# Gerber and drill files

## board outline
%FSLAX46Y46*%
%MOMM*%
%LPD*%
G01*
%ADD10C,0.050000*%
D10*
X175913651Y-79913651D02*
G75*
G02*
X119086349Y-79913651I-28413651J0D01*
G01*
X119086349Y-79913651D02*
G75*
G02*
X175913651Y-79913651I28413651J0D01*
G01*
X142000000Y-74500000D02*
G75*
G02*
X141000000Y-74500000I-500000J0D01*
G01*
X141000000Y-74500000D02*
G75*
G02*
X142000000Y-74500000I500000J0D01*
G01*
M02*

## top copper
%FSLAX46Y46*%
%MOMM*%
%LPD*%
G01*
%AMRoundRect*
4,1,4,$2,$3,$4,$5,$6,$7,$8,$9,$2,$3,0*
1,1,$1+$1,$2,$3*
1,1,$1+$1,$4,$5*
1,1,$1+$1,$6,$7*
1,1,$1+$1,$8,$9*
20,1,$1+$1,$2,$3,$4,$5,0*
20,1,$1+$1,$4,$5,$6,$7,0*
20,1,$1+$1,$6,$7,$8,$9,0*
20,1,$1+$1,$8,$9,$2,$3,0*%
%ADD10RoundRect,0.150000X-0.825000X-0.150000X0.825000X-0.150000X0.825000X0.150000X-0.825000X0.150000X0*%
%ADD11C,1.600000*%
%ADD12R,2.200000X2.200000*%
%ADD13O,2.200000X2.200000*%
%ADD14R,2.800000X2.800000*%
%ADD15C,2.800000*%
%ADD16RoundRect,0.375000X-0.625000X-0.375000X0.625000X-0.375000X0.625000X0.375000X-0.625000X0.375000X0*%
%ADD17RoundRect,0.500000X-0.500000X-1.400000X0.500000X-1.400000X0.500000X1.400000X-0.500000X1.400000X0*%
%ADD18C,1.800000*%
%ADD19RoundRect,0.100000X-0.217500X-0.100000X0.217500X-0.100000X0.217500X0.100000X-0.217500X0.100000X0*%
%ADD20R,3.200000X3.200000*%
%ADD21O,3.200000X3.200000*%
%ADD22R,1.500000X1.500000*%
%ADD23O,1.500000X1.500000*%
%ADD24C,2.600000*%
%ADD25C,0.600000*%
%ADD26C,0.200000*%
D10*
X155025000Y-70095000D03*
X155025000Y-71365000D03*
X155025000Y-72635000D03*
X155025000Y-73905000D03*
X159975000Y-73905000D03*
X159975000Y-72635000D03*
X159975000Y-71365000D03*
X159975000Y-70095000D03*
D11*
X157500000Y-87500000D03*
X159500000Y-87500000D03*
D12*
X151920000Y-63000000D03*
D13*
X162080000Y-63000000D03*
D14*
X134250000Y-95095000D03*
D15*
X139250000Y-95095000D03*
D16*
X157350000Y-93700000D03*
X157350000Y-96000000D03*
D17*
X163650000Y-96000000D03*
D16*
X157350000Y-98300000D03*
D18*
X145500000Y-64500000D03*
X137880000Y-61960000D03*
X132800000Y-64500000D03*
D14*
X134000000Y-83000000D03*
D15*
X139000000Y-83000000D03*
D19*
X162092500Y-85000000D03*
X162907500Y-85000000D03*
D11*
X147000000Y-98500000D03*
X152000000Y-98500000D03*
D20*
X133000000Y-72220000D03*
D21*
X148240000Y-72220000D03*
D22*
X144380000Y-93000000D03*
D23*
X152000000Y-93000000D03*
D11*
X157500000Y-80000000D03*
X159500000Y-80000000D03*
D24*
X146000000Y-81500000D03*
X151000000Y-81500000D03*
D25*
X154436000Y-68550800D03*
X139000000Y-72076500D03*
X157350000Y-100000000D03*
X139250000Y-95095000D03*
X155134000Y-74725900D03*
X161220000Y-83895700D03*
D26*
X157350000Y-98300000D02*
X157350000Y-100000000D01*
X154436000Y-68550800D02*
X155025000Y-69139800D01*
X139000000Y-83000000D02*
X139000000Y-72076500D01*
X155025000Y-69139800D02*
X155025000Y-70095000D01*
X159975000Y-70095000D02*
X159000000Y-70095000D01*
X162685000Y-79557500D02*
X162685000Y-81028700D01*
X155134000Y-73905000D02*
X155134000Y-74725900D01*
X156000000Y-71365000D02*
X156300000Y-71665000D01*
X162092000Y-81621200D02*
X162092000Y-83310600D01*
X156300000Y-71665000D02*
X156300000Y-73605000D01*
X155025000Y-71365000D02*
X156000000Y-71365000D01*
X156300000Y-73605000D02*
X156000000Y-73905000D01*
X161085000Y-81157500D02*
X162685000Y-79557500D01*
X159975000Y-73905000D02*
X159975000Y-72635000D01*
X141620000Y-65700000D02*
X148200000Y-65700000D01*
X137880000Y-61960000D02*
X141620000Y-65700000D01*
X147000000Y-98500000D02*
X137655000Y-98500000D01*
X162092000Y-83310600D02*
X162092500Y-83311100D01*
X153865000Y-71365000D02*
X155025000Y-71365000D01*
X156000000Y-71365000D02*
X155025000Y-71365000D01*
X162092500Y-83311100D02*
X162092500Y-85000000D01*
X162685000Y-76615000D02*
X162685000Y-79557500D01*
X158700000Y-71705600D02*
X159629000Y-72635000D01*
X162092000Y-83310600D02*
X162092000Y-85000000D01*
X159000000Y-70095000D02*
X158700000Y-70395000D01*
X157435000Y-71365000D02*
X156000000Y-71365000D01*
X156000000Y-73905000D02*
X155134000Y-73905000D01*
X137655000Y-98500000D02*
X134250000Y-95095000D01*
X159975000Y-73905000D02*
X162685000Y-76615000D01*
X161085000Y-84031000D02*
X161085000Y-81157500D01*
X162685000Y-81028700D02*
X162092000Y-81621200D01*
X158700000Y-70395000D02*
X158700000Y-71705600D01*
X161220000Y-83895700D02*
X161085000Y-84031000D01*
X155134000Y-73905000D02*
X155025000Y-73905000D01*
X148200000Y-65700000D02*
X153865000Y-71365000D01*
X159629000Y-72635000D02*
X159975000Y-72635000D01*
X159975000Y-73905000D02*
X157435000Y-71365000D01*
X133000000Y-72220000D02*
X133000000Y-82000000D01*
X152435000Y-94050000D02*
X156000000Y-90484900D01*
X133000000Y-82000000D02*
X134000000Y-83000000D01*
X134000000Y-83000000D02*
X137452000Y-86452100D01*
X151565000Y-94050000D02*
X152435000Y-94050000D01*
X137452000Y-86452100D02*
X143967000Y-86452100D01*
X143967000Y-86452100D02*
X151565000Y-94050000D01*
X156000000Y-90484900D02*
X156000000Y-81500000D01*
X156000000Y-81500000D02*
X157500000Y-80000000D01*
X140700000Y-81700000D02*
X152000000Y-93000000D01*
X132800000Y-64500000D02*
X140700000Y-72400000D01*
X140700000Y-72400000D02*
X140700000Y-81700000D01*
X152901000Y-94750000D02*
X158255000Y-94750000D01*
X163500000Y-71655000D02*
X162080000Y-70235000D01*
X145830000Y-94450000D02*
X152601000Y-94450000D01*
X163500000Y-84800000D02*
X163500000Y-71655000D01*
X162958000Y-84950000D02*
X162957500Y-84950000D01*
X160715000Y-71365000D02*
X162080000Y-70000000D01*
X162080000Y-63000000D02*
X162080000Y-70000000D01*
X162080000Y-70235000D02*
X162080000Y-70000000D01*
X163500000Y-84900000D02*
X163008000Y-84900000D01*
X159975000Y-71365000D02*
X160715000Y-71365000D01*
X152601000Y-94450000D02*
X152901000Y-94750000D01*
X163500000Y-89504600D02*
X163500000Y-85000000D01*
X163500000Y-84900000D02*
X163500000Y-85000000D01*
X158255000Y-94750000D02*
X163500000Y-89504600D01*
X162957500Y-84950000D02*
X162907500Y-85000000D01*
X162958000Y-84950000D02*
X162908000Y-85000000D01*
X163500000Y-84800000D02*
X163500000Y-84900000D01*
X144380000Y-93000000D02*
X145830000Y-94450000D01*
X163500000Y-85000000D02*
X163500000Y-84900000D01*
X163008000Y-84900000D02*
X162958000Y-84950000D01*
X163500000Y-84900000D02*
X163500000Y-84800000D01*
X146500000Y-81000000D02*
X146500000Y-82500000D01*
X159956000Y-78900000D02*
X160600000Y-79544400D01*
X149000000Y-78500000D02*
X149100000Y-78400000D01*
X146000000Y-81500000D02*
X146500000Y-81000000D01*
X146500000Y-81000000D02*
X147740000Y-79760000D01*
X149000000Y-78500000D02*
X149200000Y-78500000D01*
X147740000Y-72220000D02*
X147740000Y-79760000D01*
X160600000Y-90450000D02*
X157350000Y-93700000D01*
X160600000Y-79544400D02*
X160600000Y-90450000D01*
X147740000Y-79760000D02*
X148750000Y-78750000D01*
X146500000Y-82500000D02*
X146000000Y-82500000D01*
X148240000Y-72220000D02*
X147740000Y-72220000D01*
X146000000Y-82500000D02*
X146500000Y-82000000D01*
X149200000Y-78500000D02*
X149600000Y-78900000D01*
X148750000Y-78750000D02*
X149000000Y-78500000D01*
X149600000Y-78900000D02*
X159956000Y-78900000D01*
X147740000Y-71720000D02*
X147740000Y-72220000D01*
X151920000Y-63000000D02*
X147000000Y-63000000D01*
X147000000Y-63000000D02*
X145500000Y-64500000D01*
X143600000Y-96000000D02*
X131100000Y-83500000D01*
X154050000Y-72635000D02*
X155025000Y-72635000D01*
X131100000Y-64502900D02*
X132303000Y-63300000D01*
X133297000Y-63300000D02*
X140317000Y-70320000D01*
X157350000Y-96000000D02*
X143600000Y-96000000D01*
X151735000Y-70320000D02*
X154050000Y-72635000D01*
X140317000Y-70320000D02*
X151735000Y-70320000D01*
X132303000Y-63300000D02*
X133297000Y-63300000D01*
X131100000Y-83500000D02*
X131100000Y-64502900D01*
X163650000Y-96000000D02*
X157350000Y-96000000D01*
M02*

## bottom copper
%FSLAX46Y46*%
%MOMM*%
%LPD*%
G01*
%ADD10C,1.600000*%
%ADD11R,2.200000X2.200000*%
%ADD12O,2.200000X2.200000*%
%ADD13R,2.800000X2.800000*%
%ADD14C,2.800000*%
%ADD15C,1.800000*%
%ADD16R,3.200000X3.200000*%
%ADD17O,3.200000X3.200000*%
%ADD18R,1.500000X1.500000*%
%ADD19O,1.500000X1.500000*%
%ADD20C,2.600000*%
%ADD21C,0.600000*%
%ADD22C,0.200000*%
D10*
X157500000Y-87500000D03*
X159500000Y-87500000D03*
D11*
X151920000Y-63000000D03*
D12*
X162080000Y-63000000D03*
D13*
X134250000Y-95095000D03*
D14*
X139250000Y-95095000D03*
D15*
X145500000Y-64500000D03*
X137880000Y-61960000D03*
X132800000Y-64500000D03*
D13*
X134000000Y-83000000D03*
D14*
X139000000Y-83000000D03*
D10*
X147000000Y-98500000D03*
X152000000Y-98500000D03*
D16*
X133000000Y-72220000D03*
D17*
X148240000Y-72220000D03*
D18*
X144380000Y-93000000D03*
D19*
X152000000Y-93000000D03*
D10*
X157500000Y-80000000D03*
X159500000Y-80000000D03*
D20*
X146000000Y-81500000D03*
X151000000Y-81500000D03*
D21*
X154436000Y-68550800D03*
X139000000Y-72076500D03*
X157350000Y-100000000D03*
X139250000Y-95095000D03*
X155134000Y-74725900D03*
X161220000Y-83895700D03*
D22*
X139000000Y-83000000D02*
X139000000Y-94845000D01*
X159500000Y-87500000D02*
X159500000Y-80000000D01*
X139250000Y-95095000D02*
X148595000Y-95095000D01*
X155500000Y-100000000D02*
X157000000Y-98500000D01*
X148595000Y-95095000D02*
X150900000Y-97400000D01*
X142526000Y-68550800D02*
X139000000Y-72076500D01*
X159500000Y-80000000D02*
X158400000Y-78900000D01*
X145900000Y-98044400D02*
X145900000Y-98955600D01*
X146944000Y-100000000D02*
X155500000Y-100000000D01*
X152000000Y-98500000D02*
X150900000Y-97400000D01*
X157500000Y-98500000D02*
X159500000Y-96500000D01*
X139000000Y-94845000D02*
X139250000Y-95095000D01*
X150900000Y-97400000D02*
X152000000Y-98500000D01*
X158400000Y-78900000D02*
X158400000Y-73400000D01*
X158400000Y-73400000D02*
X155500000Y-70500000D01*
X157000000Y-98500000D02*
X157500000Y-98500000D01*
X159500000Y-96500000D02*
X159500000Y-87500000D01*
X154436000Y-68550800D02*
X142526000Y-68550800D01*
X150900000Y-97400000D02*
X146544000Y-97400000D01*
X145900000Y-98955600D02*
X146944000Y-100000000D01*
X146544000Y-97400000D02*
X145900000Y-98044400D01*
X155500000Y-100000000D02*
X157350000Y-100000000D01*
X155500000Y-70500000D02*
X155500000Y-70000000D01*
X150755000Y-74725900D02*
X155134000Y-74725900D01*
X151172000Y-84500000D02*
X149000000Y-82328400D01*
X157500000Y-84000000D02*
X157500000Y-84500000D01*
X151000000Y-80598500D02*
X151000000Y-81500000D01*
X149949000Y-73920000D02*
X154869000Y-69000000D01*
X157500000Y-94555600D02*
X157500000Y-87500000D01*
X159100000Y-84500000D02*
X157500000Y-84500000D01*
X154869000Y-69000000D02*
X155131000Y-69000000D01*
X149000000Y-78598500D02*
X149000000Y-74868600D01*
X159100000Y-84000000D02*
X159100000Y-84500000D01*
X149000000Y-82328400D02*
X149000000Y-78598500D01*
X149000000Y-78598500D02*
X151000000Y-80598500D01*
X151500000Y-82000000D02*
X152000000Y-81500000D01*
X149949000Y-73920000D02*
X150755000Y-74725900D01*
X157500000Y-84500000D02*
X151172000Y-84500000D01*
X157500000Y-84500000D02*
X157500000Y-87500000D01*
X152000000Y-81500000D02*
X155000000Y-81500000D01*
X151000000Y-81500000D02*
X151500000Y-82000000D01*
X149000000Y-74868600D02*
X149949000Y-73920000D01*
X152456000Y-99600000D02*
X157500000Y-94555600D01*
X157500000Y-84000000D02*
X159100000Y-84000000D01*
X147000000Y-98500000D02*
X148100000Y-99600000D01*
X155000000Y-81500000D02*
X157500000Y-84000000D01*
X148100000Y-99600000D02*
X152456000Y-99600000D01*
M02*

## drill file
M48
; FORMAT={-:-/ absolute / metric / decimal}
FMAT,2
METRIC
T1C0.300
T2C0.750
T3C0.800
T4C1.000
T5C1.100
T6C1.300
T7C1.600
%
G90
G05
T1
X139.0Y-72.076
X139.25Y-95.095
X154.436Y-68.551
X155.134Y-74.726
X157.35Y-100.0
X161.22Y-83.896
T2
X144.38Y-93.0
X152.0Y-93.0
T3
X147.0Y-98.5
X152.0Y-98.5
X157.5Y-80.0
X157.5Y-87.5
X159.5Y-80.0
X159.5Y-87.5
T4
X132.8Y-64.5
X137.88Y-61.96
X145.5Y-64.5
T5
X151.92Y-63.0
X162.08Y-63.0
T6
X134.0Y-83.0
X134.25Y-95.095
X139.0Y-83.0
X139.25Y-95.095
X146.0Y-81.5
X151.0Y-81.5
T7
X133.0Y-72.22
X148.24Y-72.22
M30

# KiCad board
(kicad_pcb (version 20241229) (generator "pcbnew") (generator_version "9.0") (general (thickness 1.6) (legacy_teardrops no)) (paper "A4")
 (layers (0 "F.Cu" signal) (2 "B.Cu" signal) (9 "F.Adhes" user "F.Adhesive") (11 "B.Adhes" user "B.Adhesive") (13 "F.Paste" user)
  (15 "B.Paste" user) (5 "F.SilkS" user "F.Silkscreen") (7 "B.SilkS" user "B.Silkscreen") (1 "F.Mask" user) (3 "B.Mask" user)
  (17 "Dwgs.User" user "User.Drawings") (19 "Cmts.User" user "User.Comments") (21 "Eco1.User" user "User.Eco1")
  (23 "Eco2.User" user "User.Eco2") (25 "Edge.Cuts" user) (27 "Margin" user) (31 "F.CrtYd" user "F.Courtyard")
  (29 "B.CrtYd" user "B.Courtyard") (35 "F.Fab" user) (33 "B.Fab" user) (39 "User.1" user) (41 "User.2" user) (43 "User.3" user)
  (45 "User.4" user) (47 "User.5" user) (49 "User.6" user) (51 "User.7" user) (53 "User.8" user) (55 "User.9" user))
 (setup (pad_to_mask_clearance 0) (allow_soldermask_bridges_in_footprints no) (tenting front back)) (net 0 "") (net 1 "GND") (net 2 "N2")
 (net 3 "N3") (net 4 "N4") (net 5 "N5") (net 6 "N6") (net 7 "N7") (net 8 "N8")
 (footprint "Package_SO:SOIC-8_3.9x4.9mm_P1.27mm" (layer "F.Cu") (at 157.5 72)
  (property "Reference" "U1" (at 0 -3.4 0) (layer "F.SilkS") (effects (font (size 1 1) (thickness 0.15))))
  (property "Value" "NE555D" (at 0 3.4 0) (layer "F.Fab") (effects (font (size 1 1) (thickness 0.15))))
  (pad "1" smd roundrect (at -2.475 -1.905) (size 1.95 0.6) (layers "F.Cu" "F.Mask" "F.Paste") (roundrect_rratio 0.25) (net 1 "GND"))
  (pad "2" smd roundrect (at -2.475 -0.635) (size 1.95 0.6) (layers "F.Cu" "F.Mask" "F.Paste") (roundrect_rratio 0.25) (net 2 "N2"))
  (pad "3" smd roundrect (at -2.475 0.635) (size 1.95 0.6) (layers "F.Cu" "F.Mask" "F.Paste") (roundrect_rratio 0.25) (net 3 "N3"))
  (pad "4" smd roundrect (at -2.475 1.905) (size 1.95 0.6) (layers "F.Cu" "F.Mask" "F.Paste") (roundrect_rratio 0.25) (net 2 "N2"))
  (pad "5" smd roundrect (at 2.475 1.905) (size 1.95 0.6) (layers "F.Cu" "F.Mask" "F.Paste") (roundrect_rratio 0.25) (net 2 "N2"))
  (pad "6" smd roundrect (at 2.475 0.635) (size 1.95 0.6) (layers "F.Cu" "F.Mask" "F.Paste") (roundrect_rratio 0.25) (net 2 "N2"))
  (pad "7" smd roundrect (at 2.475 -0.635) (size 1.95 0.6) (layers "F.Cu" "F.Mask" "F.Paste") (roundrect_rratio 0.25) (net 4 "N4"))
  (pad "8" smd roundrect (at 2.475 -1.905) (size 1.95 0.6) (layers "F.Cu" "F.Mask" "F.Paste") (roundrect_rratio 0.25) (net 2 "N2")))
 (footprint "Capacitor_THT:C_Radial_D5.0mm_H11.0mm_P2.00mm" (layer "F.Cu") (at 157.5 87.5)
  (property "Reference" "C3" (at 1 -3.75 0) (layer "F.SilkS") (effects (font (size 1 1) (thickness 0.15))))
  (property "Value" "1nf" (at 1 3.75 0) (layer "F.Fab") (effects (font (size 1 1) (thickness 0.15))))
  (pad "1" thru_hole circle (at 0 0) (size 1.6 1.6) (drill 0.8) (layers "*.Cu" "*.Mask") (remove_unused_layers no) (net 2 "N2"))
  (pad "2" thru_hole circle (at 2 0) (size 1.6 1.6) (drill 0.8) (layers "*.Cu" "*.Mask") (remove_unused_layers no) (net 1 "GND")))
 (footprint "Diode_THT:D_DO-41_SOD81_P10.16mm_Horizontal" (layer "F.Cu") (at 151.92 63)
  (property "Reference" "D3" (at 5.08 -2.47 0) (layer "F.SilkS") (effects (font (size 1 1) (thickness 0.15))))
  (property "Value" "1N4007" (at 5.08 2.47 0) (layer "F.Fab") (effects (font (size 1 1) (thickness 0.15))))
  (pad "1" thru_hole rect (at 0 0) (size 2.2 2.2) (drill 1.1) (layers "*.Cu" "*.Mask") (remove_unused_layers no) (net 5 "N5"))
  (pad "2" thru_hole oval (at 10.16 0) (size 2.2 2.2) (drill 1.1) (layers "*.Cu" "*.Mask") (remove_unused_layers no) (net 4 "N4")))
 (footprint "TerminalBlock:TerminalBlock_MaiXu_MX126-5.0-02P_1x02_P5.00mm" (layer "F.Cu") (at 134.25 95.095)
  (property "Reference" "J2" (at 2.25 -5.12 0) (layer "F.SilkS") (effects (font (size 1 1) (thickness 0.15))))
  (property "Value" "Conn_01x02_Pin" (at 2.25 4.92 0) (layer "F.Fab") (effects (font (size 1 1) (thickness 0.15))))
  (pad "1" thru_hole rect (at 0 0) (size 2.8 2.8) (drill 1.3) (layers "*.Cu" "*.Mask") (remove_unused_layers no) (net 2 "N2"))
  (pad "2" thru_hole circle (at 5 0) (size 2.8 2.8) (drill 1.3) (layers "*.Cu" "*.Mask") (remove_unused_layers no) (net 1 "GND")))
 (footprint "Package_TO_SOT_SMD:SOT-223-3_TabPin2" (layer "F.Cu") (at 160.5 96)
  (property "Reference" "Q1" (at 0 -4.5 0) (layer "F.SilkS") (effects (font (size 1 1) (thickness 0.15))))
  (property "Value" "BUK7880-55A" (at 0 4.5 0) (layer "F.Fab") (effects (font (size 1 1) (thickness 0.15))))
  (pad "1" smd roundrect (at -3.15 -2.3) (size 2 1.5) (layers "F.Cu" "F.Mask" "F.Paste") (roundrect_rratio 0.25) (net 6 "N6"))
  (pad "2" smd roundrect (at -3.15 0) (size 2 1.5) (layers "F.Cu" "F.Mask" "F.Paste") (roundrect_rratio 0.25) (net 3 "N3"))
  (pad "2" smd roundrect (at 3.15 0) (size 2 3.8) (layers "F.Cu" "F.Mask" "F.Paste") (roundrect_rratio 0.25) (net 3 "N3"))
  (pad "3" smd roundrect (at -3.15 2.3) (size 2 1.5) (layers "F.Cu" "F.Mask" "F.Paste") (roundrect_rratio 0.25) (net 1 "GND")))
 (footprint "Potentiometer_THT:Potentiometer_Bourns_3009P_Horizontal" (layer "F.Cu") (at 145.5 64.5)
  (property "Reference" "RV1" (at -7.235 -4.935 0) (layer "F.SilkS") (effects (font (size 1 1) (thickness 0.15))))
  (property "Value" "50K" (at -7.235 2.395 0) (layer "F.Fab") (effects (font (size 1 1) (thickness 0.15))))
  (pad "1" thru_hole circle (at 0 0) (size 1.8 1.8) (drill 1) (layers "*.Cu" "*.Mask") (remove_unused_layers no) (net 5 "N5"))
  (pad "2" thru_hole circle (at -7.62 -2.54) (size 1.8 1.8) (drill 1) (layers "*.Cu" "*.Mask") (remove_unused_layers no) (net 2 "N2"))
  (pad "3" thru_hole circle (at -12.7 0) (size 1.8 1.8) (drill 1) (layers "*.Cu" "*.Mask") (remove_unused_layers no) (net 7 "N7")))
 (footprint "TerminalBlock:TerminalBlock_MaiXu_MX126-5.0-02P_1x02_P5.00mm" (layer "F.Cu") (at 134 83)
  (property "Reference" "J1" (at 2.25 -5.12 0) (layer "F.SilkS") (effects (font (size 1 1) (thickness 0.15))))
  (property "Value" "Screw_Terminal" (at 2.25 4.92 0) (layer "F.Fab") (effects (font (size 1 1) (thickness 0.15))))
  (pad "1" thru_hole rect (at 0 0) (size 2.8 2.8) (drill 1.3) (layers "*.Cu" "*.Mask") (remove_unused_layers no) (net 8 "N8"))
  (pad "2" thru_hole circle (at 5 0) (size 2.8 2.8) (drill 1.3) (layers "*.Cu" "*.Mask") (remove_unused_layers no) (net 1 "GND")))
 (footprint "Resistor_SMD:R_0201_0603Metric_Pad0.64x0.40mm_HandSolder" (layer "F.Cu") (at 162.5 85)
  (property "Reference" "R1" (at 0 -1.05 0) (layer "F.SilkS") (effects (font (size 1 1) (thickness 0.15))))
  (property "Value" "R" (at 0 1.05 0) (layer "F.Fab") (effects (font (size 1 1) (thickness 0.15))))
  (pad "" smd roundrect (at -0.4325 0) (size 0.458 0.36) (layers "F.Paste") (roundrect_rratio 0.25))
  (pad "" smd roundrect (at 0.4325 0) (size 0.458 0.36) (layers "F.Paste") (roundrect_rratio 0.25))
  (pad "1" smd roundrect (at -0.4075 0) (size 0.635 0.4) (layers "F.Cu" "F.Mask") (roundrect_rratio 0.25) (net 2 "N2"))
  (pad "2" smd roundrect (at 0.4075 0) (size 0.635 0.4) (layers "F.Cu" "F.Mask") (roundrect_rratio 0.25) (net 4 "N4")))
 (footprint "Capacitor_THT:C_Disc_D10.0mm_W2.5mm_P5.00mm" (layer "F.Cu") (at 147 98.5)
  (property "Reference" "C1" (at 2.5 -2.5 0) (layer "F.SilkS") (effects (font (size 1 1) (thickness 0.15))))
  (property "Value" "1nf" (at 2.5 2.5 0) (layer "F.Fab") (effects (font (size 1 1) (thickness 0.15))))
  (pad "1" thru_hole circle (at 0 0) (size 1.6 1.6) (drill 0.8) (layers "*.Cu" "*.Mask") (remove_unused_layers no) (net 2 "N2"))
  (pad "2" thru_hole circle (at 5 0) (size 1.6 1.6) (drill 0.8) (layers "*.Cu" "*.Mask") (remove_unused_layers no) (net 1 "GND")))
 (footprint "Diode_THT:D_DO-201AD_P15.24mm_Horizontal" (layer "F.Cu") (at 133 72.22)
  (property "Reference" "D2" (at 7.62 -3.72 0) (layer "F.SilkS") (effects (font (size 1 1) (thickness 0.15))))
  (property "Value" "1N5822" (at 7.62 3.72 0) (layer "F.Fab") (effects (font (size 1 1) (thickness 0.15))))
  (pad "1" thru_hole rect (at 0 0) (size 3.2 3.2) (drill 1.6) (layers "*.Cu" "*.Mask") (remove_unused_layers no) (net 8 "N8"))
  (pad "2" thru_hole oval (at 15.24 0) (size 3.2 3.2) (drill 1.6) (layers "*.Cu" "*.Mask") (remove_unused_layers no) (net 6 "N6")))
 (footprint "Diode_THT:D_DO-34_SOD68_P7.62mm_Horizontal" (layer "F.Cu") (at 144.38 93)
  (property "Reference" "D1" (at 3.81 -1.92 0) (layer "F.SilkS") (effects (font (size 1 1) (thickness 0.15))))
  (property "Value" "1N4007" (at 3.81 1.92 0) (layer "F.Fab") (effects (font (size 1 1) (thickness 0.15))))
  (pad "1" thru_hole rect (at 0 0) (size 1.5 1.5) (drill 0.75) (layers "*.Cu" "*.Mask") (remove_unused_layers no) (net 4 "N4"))
  (pad "2" thru_hole oval (at 7.62 0) (size 1.5 1.5) (drill 0.75) (layers "*.Cu" "*.Mask") (remove_unused_layers no) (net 7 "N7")))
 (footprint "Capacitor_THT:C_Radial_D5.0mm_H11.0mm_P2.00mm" (layer "F.Cu") (at 157.5 80)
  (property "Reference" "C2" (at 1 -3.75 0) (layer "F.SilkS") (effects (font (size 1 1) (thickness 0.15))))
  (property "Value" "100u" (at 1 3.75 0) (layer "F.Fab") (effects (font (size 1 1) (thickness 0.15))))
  (pad "1" thru_hole circle (at 0 0) (size 1.6 1.6) (drill 0.8) (layers "*.Cu" "*.Mask") (remove_unused_layers no) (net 8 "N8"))
  (pad "2" thru_hole circle (at 2 0) (size 1.6 1.6) (drill 0.8) (layers "*.Cu" "*.Mask") (remove_unused_layers no) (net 1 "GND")))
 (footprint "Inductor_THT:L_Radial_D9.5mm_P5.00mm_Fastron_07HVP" (layer "F.Cu") (at 146 81.5)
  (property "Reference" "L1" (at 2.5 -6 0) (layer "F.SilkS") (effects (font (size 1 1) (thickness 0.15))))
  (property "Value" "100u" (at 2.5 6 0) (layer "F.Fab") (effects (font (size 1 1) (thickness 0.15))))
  (pad "1" thru_hole circle (at 0 0) (size 2.6 2.6) (drill 1.3) (layers "*.Cu" "*.Mask") (remove_unused_layers no) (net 6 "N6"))
  (pad "2" thru_hole circle (at 5 0) (size 2.6 2.6) (drill 1.3) (layers "*.Cu" "*.Mask") (remove_unused_layers no) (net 2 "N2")))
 (gr_circle (center 147.5 79.913651) (end 129.649579 57.807136) (stroke (width 0.05) (type default)) (fill no) (layer "Edge.Cuts"))
 (gr_circle (center 141.5 74.5) (end 142 74.5) (stroke (width 0.05) (type default)) (fill no) (layer "Edge.Cuts"))
 (segment (start 157.35 98.3) (end 157.35 100) (width 0.2) (layer "F.Cu") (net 1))
 (segment (start 154.436 68.5508) (end 155.025 69.1398) (width 0.2) (layer "F.Cu") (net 1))
 (segment (start 139 83) (end 139 72.0765) (width 0.2) (layer "F.Cu") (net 1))
 (segment (start 155.025 69.1398) (end 155.025 70.095) (width 0.2) (layer "F.Cu") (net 1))
 (via (at 154.436 68.5508) (size 0.6) (drill 0.3) (layers "F.Cu" "B.Cu") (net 1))
 (via (at 139 72.0765) (size 0.6) (drill 0.3) (layers "F.Cu" "B.Cu") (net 1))
 (via (at 157.35 100) (size 0.6) (drill 0.3) (layers "F.Cu" "B.Cu") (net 1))
 (via (at 139.25 95.095) (size 0.6) (drill 0.3) (layers "F.Cu" "B.Cu") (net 1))
 (segment (start 139 83) (end 139 94.845) (width 0.2) (layer "B.Cu") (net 1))
 (segment (start 159.5 87.5) (end 159.5 80) (width 0.2) (layer "B.Cu") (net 1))
 (segment (start 139.25 95.095) (end 148.595 95.095) (width 0.2) (layer "B.Cu") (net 1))
 (segment (start 155.5 100) (end 157 98.5) (width 0.2) (layer "B.Cu") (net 1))
 (segment (start 148.595 95.095) (end 150.9 97.4) (width 0.2) (layer "B.Cu") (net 1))
 (segment (start 142.526 68.5508) (end 139 72.0765) (width 0.2) (layer "B.Cu") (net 1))
 (segment (start 159.5 80) (end 158.4 78.9) (width 0.2) (layer "B.Cu") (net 1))
 (segment (start 145.9 98.0444) (end 145.9 98.9556) (width 0.2) (layer "B.Cu") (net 1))
 (segment (start 146.944 100) (end 155.5 100) (width 0.2) (layer "B.Cu") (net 1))
 (segment (start 152 98.5) (end 150.9 97.4) (width 0.2) (layer "B.Cu") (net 1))
 (segment (start 157.5 98.5) (end 159.5 96.5) (width 0.2) (layer "B.Cu") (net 1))
 (segment (start 139 94.845) (end 139.25 95.095) (width 0.2) (layer "B.Cu") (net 1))
 (segment (start 150.9 97.4) (end 152 98.5) (width 0.2) (layer "B.Cu") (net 1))
 (segment (start 158.4 78.9) (end 158.4 73.4) (width 0.2) (layer "B.Cu") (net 1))
 (segment (start 158.4 73.4) (end 155.5 70.5) (width 0.2) (layer "B.Cu") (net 1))
 (segment (start 157 98.5) (end 157.5 98.5) (width 0.2) (layer "B.Cu") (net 1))
 (segment (start 159.5 96.5) (end 159.5 87.5) (width 0.2) (layer "B.Cu") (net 1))
 (segment (start 154.436 68.5508) (end 142.526 68.5508) (width 0.2) (layer "B.Cu") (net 1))
 (segment (start 150.9 97.4) (end 146.544 97.4) (width 0.2) (layer "B.Cu") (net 1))
 (segment (start 145.9 98.9556) (end 146.944 100) (width 0.2) (layer "B.Cu") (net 1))
 (segment (start 146.544 97.4) (end 145.9 98.0444) (width 0.2) (layer "B.Cu") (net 1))
 (segment (start 155.5 100) (end 157.35 100) (width 0.2) (layer "B.Cu") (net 1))
 (segment (start 155.5 70.5) (end 155.5 70) (width 0.2) (layer "B.Cu") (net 1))
 (segment (start 159.975 70.095) (end 159 70.095) (width 0.2) (layer "F.Cu") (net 2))
 (segment (start 162.685 79.5575) (end 162.685 81.0287) (width 0.2) (layer "F.Cu") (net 2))
 (segment (start 155.134 73.905) (end 155.134 74.7259) (width 0.2) (layer "F.Cu") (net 2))
 (segment (start 156 71.365) (end 156.3 71.665) (width 0.2) (layer "F.Cu") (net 2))
 (segment (start 162.092 81.6212) (end 162.092 83.3106) (width 0.2) (layer "F.Cu") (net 2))
 (segment (start 156.3 71.665) (end 156.3 73.605) (width 0.2) (layer "F.Cu") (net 2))
 (segment (start 155.025 71.365) (end 156 71.365) (width 0.2) (layer "F.Cu") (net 2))
 (segment (start 156.3 73.605) (end 156 73.905) (width 0.2) (layer "F.Cu") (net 2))
 (segment (start 161.085 81.1575) (end 162.685 79.5575) (width 0.2) (layer "F.Cu") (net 2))
 (segment (start 159.975 73.905) (end 159.975 72.635) (width 0.2) (layer "F.Cu") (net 2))
 (segment (start 141.62 65.7) (end 148.2 65.7) (width 0.2) (layer "F.Cu") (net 2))
 (segment (start 137.88 61.96) (end 141.62 65.7) (width 0.2) (layer "F.Cu") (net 2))
 (segment (start 147 98.5) (end 137.655 98.5) (width 0.2) (layer "F.Cu") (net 2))
 (segment (start 162.092 83.3106) (end 162.0925 83.3111) (width 0.2) (layer "F.Cu") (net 2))
 (segment (start 153.865 71.365) (end 155.025 71.365) (width 0.2) (layer "F.Cu") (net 2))
 (segment (start 156 71.365) (end 155.025 71.365) (width 0.2) (layer "F.Cu") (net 2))
 (segment (start 162.0925 83.3111) (end 162.0925 85) (width 0.2) (layer "F.Cu") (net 2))
 (segment (start 162.685 76.615) (end 162.685 79.5575) (width 0.2) (layer "F.Cu") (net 2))
 (segment (start 158.7 71.7056) (end 159.629 72.635) (width 0.2) (layer "F.Cu") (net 2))
 (segment (start 162.092 83.3106) (end 162.092 85) (width 0.2) (layer "F.Cu") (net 2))
 (segment (start 159 70.095) (end 158.7 70.395) (width 0.2) (layer "F.Cu") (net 2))
 (segment (start 157.435 71.365) (end 156 71.365) (width 0.2) (layer "F.Cu") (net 2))
 (segment (start 156 73.905) (end 155.134 73.905) (width 0.2) (layer "F.Cu") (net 2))
 (segment (start 137.655 98.5) (end 134.25 95.095) (width 0.2) (layer "F.Cu") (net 2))
 (segment (start 159.975 73.905) (end 162.685 76.615) (width 0.2) (layer "F.Cu") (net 2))
 (segment (start 161.085 84.031) (end 161.085 81.1575) (width 0.2) (layer "F.Cu") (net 2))
 (segment (start 162.685 81.0287) (end 162.092 81.6212) (width 0.2) (layer "F.Cu") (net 2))
 (segment (start 158.7 70.395) (end 158.7 71.7056) (width 0.2) (layer "F.Cu") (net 2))
 (segment (start 161.22 83.8957) (end 161.085 84.031) (width 0.2) (layer "F.Cu") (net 2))
 (segment (start 155.134 73.905) (end 155.025 73.905) (width 0.2) (layer "F.Cu") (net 2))
 (segment (start 148.2 65.7) (end 153.865 71.365) (width 0.2) (layer "F.Cu") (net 2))
 (segment (start 159.629 72.635) (end 159.975 72.635) (width 0.2) (layer "F.Cu") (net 2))
 (segment (start 159.975 73.905) (end 157.435 71.365) (width 0.2) (layer "F.Cu") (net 2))
 (via (at 155.134 74.7259) (size 0.6) (drill 0.3) (layers "F.Cu" "B.Cu") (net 2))
 (via (at 161.22 83.8957) (size 0.6) (drill 0.3) (layers "F.Cu" "B.Cu") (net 2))
 (segment (start 150.755 74.7259) (end 155.134 74.7259) (width 0.2) (layer "B.Cu") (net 2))
 (segment (start 151.172 84.5) (end 149 82.3284) (width 0.2) (layer "B.Cu") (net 2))
 (segment (start 157.5 84) (end 157.5 84.5) (width 0.2) (layer "B.Cu") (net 2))
 (segment (start 151 80.5985) (end 151 81.5) (width 0.2) (layer "B.Cu") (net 2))
 (segment (start 149.949 73.92) (end 154.869 69) (width 0.2) (layer "B.Cu") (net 2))
 (segment (start 157.5 94.5556) (end 157.5 87.5) (width 0.2) (layer "B.Cu") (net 2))
 (segment (start 159.1 84.5) (end 157.5 84.5) (width 0.2) (layer "B.Cu") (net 2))
 (segment (start 154.869 69) (end 155.131 69) (width 0.2) (layer "B.Cu") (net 2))
 (segment (start 149 78.5985) (end 149 74.8686) (width 0.2) (layer "B.Cu") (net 2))
 (segment (start 159.1 84) (end 159.1 84.5) (width 0.2) (layer "B.Cu") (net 2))
 (segment (start 149 82.3284) (end 149 78.5985) (width 0.2) (layer "B.Cu") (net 2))
 (segment (start 149 78.5985) (end 151 80.5985) (width 0.2) (layer "B.Cu") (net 2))
 (segment (start 151.5 82) (end 152 81.5) (width 0.2) (layer "B.Cu") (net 2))
 (segment (start 149.949 73.92) (end 150.755 74.7259) (width 0.2) (layer "B.Cu") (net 2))
 (segment (start 157.5 84.5) (end 151.172 84.5) (width 0.2) (layer "B.Cu") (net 2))
 (segment (start 157.5 84.5) (end 157.5 87.5) (width 0.2) (layer "B.Cu") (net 2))
 (segment (start 152 81.5) (end 155 81.5) (width 0.2) (layer "B.Cu") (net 2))
 (segment (start 151 81.5) (end 151.5 82) (width 0.2) (layer "B.Cu") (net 2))
 (segment (start 149 74.8686) (end 149.949 73.92) (width 0.2) (layer "B.Cu") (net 2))
 (segment (start 152.456 99.6) (end 157.5 94.5556) (width 0.2) (layer "B.Cu") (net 2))
 (segment (start 157.5 84) (end 159.1 84) (width 0.2) (layer "B.Cu") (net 2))
 (segment (start 147 98.5) (end 148.1 99.6) (width 0.2) (layer "B.Cu") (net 2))
 (segment (start 155 81.5) (end 157.5 84) (width 0.2) (layer "B.Cu") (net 2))
 (segment (start 148.1 99.6) (end 152.456 99.6) (width 0.2) (layer "B.Cu") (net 2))
 (segment (start 133 72.22) (end 133 82) (width 0.2) (layer "F.Cu") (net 8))
 (segment (start 152.435 94.05) (end 156 90.4849) (width 0.2) (layer "F.Cu") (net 8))
 (segment (start 133 82) (end 134 83) (width 0.2) (layer "F.Cu") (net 8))
 (segment (start 134 83) (end 137.452 86.4521) (width 0.2) (layer "F.Cu") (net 8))
 (segment (start 151.565 94.05) (end 152.435 94.05) (width 0.2) (layer "F.Cu") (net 8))
 (segment (start 137.452 86.4521) (end 143.967 86.4521) (width 0.2) (layer "F.Cu") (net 8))
 (segment (start 143.967 86.4521) (end 151.565 94.05) (width 0.2) (layer "F.Cu") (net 8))
 (segment (start 156 90.4849) (end 156 81.5) (width 0.2) (layer "F.Cu") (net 8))
 (segment (start 156 81.5) (end 157.5 80) (width 0.2) (layer "F.Cu") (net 8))
 (segment (start 140.7 81.7) (end 152 93) (width 0.2) (layer "F.Cu") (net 7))
 (segment (start 132.8 64.5) (end 140.7 72.4) (width 0.2) (layer "F.Cu") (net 7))
 (segment (start 140.7 72.4) (end 140.7 81.7) (width 0.2) (layer "F.Cu") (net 7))
 (segment (start 152.901 94.75) (end 158.255 94.75) (width 0.2) (layer "F.Cu") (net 4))
 (segment (start 163.5 71.655) (end 162.08 70.235) (width 0.2) (layer "F.Cu") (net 4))
 (segment (start 145.83 94.45) (end 152.601 94.45) (width 0.2) (layer "F.Cu") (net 4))
 (segment (start 163.5 84.8) (end 163.5 71.655) (width 0.2) (layer "F.Cu") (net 4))
 (segment (start 162.958 84.95) (end 162.9575 84.95) (width 0.2) (layer "F.Cu") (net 4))
 (segment (start 160.715 71.365) (end 162.08 70) (width 0.2) (layer "F.Cu") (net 4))
 (segment (start 162.08 63) (end 162.08 70) (width 0.2) (layer "F.Cu") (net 4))
 (segment (start 162.08 70.235) (end 162.08 70) (width 0.2) (layer "F.Cu") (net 4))
 (segment (start 163.5 84.9) (end 163.008 84.9) (width 0.2) (layer "F.Cu") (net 4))
 (segment (start 159.975 71.365) (end 160.715 71.365) (width 0.2) (layer "F.Cu") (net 4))
 (segment (start 152.601 94.45) (end 152.901 94.75) (width 0.2) (layer "F.Cu") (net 4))
 (segment (start 163.5 89.5046) (end 163.5 85) (width 0.2) (layer "F.Cu") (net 4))
 (segment (start 163.5 84.9) (end 163.5 85) (width 0.2) (layer "F.Cu") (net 4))
 (segment (start 158.255 94.75) (end 163.5 89.5046) (width 0.2) (layer "F.Cu") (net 4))
 (segment (start 162.9575 84.95) (end 162.9075 85) (width 0.2) (layer "F.Cu") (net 4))
 (segment (start 162.958 84.95) (end 162.908 85) (width 0.2) (layer "F.Cu") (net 4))
 (segment (start 163.5 84.8) (end 163.5 84.9) (width 0.2) (layer "F.Cu") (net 4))
 (segment (start 144.38 93) (end 145.83 94.45) (width 0.2) (layer "F.Cu") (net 4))
 (segment (start 163.5 85) (end 163.5 84.9) (width 0.2) (layer "F.Cu") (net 4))
 (segment (start 163.008 84.9) (end 162.958 84.95) (width 0.2) (layer "F.Cu") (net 4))
 (segment (start 163.5 84.9) (end 163.5 84.8) (width 0.2) (layer "F.Cu") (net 4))
 (segment (start 146.5 81) (end 146.5 82.5) (width 0.2) (layer "F.Cu") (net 6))
 (segment (start 159.956 78.9) (end 160.6 79.5444) (width 0.2) (layer "F.Cu") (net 6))
 (segment (start 149 78.5) (end 149.1 78.4) (width 0.2) (layer "F.Cu") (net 6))
 (segment (start 146 81.5) (end 146.5 81) (width 0.2) (layer "F.Cu") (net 6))
 (segment (start 146.5 81) (end 147.74 79.76) (width 0.2) (layer "F.Cu") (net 6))
 (segment (start 149 78.5) (end 149.2 78.5) (width 0.2) (layer "F.Cu") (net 6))
 (segment (start 147.74 72.22) (end 147.74 79.76) (width 0.2) (layer "F.Cu") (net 6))
 (segment (start 160.6 90.45) (end 157.35 93.7) (width 0.2) (layer "F.Cu") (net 6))
 (segment (start 160.6 79.5444) (end 160.6 90.45) (width 0.2) (layer "F.Cu") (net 6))
 (segment (start 147.74 79.76) (end 148.75 78.75) (width 0.2) (layer "F.Cu") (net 6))
 (segment (start 146.5 82.5) (end 146 82.5) (width 0.2) (layer "F.Cu") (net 6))
 (segment (start 148.24 72.22) (end 147.74 72.22) (width 0.2) (layer "F.Cu") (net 6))
 (segment (start 146 82.5) (end 146.5 82) (width 0.2) (layer "F.Cu") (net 6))
 (segment (start 149.2 78.5) (end 149.6 78.9) (width 0.2) (layer "F.Cu") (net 6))
 (segment (start 148.75 78.75) (end 149 78.5) (width 0.2) (layer "F.Cu") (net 6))
 (segment (start 149.6 78.9) (end 159.956 78.9) (width 0.2) (layer "F.Cu") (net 6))
 (segment (start 147.74 71.72) (end 147.74 72.22) (width 0.2) (layer "F.Cu") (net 6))
 (segment (start 151.92 63) (end 147 63) (width 0.2) (layer "F.Cu") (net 5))
 (segment (start 147 63) (end 145.5 64.5) (width 0.2) (layer "F.Cu") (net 5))
 (segment (start 143.6 96) (end 131.1 83.5) (width 0.2) (layer "F.Cu") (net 3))
 (segment (start 154.05 72.635) (end 155.025 72.635) (width 0.2) (layer "F.Cu") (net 3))
 (segment (start 131.1 64.5029) (end 132.303 63.3) (width 0.2) (layer "F.Cu") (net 3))
 (segment (start 133.297 63.3) (end 140.317 70.32) (width 0.2) (layer "F.Cu") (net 3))
 (segment (start 157.35 96) (end 143.6 96) (width 0.2) (layer "F.Cu") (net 3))
 (segment (start 151.735 70.32) (end 154.05 72.635) (width 0.2) (layer "F.Cu") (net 3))
 (segment (start 140.317 70.32) (end 151.735 70.32) (width 0.2) (layer "F.Cu") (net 3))
 (segment (start 132.303 63.3) (end 133.297 63.3) (width 0.2) (layer "F.Cu") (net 3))
 (segment (start 131.1 83.5) (end 131.1 64.5029) (width 0.2) (layer "F.Cu") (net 3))
 (segment (start 163.65 96) (end 157.35 96) (width 0.2) (layer "F.Cu") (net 3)))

